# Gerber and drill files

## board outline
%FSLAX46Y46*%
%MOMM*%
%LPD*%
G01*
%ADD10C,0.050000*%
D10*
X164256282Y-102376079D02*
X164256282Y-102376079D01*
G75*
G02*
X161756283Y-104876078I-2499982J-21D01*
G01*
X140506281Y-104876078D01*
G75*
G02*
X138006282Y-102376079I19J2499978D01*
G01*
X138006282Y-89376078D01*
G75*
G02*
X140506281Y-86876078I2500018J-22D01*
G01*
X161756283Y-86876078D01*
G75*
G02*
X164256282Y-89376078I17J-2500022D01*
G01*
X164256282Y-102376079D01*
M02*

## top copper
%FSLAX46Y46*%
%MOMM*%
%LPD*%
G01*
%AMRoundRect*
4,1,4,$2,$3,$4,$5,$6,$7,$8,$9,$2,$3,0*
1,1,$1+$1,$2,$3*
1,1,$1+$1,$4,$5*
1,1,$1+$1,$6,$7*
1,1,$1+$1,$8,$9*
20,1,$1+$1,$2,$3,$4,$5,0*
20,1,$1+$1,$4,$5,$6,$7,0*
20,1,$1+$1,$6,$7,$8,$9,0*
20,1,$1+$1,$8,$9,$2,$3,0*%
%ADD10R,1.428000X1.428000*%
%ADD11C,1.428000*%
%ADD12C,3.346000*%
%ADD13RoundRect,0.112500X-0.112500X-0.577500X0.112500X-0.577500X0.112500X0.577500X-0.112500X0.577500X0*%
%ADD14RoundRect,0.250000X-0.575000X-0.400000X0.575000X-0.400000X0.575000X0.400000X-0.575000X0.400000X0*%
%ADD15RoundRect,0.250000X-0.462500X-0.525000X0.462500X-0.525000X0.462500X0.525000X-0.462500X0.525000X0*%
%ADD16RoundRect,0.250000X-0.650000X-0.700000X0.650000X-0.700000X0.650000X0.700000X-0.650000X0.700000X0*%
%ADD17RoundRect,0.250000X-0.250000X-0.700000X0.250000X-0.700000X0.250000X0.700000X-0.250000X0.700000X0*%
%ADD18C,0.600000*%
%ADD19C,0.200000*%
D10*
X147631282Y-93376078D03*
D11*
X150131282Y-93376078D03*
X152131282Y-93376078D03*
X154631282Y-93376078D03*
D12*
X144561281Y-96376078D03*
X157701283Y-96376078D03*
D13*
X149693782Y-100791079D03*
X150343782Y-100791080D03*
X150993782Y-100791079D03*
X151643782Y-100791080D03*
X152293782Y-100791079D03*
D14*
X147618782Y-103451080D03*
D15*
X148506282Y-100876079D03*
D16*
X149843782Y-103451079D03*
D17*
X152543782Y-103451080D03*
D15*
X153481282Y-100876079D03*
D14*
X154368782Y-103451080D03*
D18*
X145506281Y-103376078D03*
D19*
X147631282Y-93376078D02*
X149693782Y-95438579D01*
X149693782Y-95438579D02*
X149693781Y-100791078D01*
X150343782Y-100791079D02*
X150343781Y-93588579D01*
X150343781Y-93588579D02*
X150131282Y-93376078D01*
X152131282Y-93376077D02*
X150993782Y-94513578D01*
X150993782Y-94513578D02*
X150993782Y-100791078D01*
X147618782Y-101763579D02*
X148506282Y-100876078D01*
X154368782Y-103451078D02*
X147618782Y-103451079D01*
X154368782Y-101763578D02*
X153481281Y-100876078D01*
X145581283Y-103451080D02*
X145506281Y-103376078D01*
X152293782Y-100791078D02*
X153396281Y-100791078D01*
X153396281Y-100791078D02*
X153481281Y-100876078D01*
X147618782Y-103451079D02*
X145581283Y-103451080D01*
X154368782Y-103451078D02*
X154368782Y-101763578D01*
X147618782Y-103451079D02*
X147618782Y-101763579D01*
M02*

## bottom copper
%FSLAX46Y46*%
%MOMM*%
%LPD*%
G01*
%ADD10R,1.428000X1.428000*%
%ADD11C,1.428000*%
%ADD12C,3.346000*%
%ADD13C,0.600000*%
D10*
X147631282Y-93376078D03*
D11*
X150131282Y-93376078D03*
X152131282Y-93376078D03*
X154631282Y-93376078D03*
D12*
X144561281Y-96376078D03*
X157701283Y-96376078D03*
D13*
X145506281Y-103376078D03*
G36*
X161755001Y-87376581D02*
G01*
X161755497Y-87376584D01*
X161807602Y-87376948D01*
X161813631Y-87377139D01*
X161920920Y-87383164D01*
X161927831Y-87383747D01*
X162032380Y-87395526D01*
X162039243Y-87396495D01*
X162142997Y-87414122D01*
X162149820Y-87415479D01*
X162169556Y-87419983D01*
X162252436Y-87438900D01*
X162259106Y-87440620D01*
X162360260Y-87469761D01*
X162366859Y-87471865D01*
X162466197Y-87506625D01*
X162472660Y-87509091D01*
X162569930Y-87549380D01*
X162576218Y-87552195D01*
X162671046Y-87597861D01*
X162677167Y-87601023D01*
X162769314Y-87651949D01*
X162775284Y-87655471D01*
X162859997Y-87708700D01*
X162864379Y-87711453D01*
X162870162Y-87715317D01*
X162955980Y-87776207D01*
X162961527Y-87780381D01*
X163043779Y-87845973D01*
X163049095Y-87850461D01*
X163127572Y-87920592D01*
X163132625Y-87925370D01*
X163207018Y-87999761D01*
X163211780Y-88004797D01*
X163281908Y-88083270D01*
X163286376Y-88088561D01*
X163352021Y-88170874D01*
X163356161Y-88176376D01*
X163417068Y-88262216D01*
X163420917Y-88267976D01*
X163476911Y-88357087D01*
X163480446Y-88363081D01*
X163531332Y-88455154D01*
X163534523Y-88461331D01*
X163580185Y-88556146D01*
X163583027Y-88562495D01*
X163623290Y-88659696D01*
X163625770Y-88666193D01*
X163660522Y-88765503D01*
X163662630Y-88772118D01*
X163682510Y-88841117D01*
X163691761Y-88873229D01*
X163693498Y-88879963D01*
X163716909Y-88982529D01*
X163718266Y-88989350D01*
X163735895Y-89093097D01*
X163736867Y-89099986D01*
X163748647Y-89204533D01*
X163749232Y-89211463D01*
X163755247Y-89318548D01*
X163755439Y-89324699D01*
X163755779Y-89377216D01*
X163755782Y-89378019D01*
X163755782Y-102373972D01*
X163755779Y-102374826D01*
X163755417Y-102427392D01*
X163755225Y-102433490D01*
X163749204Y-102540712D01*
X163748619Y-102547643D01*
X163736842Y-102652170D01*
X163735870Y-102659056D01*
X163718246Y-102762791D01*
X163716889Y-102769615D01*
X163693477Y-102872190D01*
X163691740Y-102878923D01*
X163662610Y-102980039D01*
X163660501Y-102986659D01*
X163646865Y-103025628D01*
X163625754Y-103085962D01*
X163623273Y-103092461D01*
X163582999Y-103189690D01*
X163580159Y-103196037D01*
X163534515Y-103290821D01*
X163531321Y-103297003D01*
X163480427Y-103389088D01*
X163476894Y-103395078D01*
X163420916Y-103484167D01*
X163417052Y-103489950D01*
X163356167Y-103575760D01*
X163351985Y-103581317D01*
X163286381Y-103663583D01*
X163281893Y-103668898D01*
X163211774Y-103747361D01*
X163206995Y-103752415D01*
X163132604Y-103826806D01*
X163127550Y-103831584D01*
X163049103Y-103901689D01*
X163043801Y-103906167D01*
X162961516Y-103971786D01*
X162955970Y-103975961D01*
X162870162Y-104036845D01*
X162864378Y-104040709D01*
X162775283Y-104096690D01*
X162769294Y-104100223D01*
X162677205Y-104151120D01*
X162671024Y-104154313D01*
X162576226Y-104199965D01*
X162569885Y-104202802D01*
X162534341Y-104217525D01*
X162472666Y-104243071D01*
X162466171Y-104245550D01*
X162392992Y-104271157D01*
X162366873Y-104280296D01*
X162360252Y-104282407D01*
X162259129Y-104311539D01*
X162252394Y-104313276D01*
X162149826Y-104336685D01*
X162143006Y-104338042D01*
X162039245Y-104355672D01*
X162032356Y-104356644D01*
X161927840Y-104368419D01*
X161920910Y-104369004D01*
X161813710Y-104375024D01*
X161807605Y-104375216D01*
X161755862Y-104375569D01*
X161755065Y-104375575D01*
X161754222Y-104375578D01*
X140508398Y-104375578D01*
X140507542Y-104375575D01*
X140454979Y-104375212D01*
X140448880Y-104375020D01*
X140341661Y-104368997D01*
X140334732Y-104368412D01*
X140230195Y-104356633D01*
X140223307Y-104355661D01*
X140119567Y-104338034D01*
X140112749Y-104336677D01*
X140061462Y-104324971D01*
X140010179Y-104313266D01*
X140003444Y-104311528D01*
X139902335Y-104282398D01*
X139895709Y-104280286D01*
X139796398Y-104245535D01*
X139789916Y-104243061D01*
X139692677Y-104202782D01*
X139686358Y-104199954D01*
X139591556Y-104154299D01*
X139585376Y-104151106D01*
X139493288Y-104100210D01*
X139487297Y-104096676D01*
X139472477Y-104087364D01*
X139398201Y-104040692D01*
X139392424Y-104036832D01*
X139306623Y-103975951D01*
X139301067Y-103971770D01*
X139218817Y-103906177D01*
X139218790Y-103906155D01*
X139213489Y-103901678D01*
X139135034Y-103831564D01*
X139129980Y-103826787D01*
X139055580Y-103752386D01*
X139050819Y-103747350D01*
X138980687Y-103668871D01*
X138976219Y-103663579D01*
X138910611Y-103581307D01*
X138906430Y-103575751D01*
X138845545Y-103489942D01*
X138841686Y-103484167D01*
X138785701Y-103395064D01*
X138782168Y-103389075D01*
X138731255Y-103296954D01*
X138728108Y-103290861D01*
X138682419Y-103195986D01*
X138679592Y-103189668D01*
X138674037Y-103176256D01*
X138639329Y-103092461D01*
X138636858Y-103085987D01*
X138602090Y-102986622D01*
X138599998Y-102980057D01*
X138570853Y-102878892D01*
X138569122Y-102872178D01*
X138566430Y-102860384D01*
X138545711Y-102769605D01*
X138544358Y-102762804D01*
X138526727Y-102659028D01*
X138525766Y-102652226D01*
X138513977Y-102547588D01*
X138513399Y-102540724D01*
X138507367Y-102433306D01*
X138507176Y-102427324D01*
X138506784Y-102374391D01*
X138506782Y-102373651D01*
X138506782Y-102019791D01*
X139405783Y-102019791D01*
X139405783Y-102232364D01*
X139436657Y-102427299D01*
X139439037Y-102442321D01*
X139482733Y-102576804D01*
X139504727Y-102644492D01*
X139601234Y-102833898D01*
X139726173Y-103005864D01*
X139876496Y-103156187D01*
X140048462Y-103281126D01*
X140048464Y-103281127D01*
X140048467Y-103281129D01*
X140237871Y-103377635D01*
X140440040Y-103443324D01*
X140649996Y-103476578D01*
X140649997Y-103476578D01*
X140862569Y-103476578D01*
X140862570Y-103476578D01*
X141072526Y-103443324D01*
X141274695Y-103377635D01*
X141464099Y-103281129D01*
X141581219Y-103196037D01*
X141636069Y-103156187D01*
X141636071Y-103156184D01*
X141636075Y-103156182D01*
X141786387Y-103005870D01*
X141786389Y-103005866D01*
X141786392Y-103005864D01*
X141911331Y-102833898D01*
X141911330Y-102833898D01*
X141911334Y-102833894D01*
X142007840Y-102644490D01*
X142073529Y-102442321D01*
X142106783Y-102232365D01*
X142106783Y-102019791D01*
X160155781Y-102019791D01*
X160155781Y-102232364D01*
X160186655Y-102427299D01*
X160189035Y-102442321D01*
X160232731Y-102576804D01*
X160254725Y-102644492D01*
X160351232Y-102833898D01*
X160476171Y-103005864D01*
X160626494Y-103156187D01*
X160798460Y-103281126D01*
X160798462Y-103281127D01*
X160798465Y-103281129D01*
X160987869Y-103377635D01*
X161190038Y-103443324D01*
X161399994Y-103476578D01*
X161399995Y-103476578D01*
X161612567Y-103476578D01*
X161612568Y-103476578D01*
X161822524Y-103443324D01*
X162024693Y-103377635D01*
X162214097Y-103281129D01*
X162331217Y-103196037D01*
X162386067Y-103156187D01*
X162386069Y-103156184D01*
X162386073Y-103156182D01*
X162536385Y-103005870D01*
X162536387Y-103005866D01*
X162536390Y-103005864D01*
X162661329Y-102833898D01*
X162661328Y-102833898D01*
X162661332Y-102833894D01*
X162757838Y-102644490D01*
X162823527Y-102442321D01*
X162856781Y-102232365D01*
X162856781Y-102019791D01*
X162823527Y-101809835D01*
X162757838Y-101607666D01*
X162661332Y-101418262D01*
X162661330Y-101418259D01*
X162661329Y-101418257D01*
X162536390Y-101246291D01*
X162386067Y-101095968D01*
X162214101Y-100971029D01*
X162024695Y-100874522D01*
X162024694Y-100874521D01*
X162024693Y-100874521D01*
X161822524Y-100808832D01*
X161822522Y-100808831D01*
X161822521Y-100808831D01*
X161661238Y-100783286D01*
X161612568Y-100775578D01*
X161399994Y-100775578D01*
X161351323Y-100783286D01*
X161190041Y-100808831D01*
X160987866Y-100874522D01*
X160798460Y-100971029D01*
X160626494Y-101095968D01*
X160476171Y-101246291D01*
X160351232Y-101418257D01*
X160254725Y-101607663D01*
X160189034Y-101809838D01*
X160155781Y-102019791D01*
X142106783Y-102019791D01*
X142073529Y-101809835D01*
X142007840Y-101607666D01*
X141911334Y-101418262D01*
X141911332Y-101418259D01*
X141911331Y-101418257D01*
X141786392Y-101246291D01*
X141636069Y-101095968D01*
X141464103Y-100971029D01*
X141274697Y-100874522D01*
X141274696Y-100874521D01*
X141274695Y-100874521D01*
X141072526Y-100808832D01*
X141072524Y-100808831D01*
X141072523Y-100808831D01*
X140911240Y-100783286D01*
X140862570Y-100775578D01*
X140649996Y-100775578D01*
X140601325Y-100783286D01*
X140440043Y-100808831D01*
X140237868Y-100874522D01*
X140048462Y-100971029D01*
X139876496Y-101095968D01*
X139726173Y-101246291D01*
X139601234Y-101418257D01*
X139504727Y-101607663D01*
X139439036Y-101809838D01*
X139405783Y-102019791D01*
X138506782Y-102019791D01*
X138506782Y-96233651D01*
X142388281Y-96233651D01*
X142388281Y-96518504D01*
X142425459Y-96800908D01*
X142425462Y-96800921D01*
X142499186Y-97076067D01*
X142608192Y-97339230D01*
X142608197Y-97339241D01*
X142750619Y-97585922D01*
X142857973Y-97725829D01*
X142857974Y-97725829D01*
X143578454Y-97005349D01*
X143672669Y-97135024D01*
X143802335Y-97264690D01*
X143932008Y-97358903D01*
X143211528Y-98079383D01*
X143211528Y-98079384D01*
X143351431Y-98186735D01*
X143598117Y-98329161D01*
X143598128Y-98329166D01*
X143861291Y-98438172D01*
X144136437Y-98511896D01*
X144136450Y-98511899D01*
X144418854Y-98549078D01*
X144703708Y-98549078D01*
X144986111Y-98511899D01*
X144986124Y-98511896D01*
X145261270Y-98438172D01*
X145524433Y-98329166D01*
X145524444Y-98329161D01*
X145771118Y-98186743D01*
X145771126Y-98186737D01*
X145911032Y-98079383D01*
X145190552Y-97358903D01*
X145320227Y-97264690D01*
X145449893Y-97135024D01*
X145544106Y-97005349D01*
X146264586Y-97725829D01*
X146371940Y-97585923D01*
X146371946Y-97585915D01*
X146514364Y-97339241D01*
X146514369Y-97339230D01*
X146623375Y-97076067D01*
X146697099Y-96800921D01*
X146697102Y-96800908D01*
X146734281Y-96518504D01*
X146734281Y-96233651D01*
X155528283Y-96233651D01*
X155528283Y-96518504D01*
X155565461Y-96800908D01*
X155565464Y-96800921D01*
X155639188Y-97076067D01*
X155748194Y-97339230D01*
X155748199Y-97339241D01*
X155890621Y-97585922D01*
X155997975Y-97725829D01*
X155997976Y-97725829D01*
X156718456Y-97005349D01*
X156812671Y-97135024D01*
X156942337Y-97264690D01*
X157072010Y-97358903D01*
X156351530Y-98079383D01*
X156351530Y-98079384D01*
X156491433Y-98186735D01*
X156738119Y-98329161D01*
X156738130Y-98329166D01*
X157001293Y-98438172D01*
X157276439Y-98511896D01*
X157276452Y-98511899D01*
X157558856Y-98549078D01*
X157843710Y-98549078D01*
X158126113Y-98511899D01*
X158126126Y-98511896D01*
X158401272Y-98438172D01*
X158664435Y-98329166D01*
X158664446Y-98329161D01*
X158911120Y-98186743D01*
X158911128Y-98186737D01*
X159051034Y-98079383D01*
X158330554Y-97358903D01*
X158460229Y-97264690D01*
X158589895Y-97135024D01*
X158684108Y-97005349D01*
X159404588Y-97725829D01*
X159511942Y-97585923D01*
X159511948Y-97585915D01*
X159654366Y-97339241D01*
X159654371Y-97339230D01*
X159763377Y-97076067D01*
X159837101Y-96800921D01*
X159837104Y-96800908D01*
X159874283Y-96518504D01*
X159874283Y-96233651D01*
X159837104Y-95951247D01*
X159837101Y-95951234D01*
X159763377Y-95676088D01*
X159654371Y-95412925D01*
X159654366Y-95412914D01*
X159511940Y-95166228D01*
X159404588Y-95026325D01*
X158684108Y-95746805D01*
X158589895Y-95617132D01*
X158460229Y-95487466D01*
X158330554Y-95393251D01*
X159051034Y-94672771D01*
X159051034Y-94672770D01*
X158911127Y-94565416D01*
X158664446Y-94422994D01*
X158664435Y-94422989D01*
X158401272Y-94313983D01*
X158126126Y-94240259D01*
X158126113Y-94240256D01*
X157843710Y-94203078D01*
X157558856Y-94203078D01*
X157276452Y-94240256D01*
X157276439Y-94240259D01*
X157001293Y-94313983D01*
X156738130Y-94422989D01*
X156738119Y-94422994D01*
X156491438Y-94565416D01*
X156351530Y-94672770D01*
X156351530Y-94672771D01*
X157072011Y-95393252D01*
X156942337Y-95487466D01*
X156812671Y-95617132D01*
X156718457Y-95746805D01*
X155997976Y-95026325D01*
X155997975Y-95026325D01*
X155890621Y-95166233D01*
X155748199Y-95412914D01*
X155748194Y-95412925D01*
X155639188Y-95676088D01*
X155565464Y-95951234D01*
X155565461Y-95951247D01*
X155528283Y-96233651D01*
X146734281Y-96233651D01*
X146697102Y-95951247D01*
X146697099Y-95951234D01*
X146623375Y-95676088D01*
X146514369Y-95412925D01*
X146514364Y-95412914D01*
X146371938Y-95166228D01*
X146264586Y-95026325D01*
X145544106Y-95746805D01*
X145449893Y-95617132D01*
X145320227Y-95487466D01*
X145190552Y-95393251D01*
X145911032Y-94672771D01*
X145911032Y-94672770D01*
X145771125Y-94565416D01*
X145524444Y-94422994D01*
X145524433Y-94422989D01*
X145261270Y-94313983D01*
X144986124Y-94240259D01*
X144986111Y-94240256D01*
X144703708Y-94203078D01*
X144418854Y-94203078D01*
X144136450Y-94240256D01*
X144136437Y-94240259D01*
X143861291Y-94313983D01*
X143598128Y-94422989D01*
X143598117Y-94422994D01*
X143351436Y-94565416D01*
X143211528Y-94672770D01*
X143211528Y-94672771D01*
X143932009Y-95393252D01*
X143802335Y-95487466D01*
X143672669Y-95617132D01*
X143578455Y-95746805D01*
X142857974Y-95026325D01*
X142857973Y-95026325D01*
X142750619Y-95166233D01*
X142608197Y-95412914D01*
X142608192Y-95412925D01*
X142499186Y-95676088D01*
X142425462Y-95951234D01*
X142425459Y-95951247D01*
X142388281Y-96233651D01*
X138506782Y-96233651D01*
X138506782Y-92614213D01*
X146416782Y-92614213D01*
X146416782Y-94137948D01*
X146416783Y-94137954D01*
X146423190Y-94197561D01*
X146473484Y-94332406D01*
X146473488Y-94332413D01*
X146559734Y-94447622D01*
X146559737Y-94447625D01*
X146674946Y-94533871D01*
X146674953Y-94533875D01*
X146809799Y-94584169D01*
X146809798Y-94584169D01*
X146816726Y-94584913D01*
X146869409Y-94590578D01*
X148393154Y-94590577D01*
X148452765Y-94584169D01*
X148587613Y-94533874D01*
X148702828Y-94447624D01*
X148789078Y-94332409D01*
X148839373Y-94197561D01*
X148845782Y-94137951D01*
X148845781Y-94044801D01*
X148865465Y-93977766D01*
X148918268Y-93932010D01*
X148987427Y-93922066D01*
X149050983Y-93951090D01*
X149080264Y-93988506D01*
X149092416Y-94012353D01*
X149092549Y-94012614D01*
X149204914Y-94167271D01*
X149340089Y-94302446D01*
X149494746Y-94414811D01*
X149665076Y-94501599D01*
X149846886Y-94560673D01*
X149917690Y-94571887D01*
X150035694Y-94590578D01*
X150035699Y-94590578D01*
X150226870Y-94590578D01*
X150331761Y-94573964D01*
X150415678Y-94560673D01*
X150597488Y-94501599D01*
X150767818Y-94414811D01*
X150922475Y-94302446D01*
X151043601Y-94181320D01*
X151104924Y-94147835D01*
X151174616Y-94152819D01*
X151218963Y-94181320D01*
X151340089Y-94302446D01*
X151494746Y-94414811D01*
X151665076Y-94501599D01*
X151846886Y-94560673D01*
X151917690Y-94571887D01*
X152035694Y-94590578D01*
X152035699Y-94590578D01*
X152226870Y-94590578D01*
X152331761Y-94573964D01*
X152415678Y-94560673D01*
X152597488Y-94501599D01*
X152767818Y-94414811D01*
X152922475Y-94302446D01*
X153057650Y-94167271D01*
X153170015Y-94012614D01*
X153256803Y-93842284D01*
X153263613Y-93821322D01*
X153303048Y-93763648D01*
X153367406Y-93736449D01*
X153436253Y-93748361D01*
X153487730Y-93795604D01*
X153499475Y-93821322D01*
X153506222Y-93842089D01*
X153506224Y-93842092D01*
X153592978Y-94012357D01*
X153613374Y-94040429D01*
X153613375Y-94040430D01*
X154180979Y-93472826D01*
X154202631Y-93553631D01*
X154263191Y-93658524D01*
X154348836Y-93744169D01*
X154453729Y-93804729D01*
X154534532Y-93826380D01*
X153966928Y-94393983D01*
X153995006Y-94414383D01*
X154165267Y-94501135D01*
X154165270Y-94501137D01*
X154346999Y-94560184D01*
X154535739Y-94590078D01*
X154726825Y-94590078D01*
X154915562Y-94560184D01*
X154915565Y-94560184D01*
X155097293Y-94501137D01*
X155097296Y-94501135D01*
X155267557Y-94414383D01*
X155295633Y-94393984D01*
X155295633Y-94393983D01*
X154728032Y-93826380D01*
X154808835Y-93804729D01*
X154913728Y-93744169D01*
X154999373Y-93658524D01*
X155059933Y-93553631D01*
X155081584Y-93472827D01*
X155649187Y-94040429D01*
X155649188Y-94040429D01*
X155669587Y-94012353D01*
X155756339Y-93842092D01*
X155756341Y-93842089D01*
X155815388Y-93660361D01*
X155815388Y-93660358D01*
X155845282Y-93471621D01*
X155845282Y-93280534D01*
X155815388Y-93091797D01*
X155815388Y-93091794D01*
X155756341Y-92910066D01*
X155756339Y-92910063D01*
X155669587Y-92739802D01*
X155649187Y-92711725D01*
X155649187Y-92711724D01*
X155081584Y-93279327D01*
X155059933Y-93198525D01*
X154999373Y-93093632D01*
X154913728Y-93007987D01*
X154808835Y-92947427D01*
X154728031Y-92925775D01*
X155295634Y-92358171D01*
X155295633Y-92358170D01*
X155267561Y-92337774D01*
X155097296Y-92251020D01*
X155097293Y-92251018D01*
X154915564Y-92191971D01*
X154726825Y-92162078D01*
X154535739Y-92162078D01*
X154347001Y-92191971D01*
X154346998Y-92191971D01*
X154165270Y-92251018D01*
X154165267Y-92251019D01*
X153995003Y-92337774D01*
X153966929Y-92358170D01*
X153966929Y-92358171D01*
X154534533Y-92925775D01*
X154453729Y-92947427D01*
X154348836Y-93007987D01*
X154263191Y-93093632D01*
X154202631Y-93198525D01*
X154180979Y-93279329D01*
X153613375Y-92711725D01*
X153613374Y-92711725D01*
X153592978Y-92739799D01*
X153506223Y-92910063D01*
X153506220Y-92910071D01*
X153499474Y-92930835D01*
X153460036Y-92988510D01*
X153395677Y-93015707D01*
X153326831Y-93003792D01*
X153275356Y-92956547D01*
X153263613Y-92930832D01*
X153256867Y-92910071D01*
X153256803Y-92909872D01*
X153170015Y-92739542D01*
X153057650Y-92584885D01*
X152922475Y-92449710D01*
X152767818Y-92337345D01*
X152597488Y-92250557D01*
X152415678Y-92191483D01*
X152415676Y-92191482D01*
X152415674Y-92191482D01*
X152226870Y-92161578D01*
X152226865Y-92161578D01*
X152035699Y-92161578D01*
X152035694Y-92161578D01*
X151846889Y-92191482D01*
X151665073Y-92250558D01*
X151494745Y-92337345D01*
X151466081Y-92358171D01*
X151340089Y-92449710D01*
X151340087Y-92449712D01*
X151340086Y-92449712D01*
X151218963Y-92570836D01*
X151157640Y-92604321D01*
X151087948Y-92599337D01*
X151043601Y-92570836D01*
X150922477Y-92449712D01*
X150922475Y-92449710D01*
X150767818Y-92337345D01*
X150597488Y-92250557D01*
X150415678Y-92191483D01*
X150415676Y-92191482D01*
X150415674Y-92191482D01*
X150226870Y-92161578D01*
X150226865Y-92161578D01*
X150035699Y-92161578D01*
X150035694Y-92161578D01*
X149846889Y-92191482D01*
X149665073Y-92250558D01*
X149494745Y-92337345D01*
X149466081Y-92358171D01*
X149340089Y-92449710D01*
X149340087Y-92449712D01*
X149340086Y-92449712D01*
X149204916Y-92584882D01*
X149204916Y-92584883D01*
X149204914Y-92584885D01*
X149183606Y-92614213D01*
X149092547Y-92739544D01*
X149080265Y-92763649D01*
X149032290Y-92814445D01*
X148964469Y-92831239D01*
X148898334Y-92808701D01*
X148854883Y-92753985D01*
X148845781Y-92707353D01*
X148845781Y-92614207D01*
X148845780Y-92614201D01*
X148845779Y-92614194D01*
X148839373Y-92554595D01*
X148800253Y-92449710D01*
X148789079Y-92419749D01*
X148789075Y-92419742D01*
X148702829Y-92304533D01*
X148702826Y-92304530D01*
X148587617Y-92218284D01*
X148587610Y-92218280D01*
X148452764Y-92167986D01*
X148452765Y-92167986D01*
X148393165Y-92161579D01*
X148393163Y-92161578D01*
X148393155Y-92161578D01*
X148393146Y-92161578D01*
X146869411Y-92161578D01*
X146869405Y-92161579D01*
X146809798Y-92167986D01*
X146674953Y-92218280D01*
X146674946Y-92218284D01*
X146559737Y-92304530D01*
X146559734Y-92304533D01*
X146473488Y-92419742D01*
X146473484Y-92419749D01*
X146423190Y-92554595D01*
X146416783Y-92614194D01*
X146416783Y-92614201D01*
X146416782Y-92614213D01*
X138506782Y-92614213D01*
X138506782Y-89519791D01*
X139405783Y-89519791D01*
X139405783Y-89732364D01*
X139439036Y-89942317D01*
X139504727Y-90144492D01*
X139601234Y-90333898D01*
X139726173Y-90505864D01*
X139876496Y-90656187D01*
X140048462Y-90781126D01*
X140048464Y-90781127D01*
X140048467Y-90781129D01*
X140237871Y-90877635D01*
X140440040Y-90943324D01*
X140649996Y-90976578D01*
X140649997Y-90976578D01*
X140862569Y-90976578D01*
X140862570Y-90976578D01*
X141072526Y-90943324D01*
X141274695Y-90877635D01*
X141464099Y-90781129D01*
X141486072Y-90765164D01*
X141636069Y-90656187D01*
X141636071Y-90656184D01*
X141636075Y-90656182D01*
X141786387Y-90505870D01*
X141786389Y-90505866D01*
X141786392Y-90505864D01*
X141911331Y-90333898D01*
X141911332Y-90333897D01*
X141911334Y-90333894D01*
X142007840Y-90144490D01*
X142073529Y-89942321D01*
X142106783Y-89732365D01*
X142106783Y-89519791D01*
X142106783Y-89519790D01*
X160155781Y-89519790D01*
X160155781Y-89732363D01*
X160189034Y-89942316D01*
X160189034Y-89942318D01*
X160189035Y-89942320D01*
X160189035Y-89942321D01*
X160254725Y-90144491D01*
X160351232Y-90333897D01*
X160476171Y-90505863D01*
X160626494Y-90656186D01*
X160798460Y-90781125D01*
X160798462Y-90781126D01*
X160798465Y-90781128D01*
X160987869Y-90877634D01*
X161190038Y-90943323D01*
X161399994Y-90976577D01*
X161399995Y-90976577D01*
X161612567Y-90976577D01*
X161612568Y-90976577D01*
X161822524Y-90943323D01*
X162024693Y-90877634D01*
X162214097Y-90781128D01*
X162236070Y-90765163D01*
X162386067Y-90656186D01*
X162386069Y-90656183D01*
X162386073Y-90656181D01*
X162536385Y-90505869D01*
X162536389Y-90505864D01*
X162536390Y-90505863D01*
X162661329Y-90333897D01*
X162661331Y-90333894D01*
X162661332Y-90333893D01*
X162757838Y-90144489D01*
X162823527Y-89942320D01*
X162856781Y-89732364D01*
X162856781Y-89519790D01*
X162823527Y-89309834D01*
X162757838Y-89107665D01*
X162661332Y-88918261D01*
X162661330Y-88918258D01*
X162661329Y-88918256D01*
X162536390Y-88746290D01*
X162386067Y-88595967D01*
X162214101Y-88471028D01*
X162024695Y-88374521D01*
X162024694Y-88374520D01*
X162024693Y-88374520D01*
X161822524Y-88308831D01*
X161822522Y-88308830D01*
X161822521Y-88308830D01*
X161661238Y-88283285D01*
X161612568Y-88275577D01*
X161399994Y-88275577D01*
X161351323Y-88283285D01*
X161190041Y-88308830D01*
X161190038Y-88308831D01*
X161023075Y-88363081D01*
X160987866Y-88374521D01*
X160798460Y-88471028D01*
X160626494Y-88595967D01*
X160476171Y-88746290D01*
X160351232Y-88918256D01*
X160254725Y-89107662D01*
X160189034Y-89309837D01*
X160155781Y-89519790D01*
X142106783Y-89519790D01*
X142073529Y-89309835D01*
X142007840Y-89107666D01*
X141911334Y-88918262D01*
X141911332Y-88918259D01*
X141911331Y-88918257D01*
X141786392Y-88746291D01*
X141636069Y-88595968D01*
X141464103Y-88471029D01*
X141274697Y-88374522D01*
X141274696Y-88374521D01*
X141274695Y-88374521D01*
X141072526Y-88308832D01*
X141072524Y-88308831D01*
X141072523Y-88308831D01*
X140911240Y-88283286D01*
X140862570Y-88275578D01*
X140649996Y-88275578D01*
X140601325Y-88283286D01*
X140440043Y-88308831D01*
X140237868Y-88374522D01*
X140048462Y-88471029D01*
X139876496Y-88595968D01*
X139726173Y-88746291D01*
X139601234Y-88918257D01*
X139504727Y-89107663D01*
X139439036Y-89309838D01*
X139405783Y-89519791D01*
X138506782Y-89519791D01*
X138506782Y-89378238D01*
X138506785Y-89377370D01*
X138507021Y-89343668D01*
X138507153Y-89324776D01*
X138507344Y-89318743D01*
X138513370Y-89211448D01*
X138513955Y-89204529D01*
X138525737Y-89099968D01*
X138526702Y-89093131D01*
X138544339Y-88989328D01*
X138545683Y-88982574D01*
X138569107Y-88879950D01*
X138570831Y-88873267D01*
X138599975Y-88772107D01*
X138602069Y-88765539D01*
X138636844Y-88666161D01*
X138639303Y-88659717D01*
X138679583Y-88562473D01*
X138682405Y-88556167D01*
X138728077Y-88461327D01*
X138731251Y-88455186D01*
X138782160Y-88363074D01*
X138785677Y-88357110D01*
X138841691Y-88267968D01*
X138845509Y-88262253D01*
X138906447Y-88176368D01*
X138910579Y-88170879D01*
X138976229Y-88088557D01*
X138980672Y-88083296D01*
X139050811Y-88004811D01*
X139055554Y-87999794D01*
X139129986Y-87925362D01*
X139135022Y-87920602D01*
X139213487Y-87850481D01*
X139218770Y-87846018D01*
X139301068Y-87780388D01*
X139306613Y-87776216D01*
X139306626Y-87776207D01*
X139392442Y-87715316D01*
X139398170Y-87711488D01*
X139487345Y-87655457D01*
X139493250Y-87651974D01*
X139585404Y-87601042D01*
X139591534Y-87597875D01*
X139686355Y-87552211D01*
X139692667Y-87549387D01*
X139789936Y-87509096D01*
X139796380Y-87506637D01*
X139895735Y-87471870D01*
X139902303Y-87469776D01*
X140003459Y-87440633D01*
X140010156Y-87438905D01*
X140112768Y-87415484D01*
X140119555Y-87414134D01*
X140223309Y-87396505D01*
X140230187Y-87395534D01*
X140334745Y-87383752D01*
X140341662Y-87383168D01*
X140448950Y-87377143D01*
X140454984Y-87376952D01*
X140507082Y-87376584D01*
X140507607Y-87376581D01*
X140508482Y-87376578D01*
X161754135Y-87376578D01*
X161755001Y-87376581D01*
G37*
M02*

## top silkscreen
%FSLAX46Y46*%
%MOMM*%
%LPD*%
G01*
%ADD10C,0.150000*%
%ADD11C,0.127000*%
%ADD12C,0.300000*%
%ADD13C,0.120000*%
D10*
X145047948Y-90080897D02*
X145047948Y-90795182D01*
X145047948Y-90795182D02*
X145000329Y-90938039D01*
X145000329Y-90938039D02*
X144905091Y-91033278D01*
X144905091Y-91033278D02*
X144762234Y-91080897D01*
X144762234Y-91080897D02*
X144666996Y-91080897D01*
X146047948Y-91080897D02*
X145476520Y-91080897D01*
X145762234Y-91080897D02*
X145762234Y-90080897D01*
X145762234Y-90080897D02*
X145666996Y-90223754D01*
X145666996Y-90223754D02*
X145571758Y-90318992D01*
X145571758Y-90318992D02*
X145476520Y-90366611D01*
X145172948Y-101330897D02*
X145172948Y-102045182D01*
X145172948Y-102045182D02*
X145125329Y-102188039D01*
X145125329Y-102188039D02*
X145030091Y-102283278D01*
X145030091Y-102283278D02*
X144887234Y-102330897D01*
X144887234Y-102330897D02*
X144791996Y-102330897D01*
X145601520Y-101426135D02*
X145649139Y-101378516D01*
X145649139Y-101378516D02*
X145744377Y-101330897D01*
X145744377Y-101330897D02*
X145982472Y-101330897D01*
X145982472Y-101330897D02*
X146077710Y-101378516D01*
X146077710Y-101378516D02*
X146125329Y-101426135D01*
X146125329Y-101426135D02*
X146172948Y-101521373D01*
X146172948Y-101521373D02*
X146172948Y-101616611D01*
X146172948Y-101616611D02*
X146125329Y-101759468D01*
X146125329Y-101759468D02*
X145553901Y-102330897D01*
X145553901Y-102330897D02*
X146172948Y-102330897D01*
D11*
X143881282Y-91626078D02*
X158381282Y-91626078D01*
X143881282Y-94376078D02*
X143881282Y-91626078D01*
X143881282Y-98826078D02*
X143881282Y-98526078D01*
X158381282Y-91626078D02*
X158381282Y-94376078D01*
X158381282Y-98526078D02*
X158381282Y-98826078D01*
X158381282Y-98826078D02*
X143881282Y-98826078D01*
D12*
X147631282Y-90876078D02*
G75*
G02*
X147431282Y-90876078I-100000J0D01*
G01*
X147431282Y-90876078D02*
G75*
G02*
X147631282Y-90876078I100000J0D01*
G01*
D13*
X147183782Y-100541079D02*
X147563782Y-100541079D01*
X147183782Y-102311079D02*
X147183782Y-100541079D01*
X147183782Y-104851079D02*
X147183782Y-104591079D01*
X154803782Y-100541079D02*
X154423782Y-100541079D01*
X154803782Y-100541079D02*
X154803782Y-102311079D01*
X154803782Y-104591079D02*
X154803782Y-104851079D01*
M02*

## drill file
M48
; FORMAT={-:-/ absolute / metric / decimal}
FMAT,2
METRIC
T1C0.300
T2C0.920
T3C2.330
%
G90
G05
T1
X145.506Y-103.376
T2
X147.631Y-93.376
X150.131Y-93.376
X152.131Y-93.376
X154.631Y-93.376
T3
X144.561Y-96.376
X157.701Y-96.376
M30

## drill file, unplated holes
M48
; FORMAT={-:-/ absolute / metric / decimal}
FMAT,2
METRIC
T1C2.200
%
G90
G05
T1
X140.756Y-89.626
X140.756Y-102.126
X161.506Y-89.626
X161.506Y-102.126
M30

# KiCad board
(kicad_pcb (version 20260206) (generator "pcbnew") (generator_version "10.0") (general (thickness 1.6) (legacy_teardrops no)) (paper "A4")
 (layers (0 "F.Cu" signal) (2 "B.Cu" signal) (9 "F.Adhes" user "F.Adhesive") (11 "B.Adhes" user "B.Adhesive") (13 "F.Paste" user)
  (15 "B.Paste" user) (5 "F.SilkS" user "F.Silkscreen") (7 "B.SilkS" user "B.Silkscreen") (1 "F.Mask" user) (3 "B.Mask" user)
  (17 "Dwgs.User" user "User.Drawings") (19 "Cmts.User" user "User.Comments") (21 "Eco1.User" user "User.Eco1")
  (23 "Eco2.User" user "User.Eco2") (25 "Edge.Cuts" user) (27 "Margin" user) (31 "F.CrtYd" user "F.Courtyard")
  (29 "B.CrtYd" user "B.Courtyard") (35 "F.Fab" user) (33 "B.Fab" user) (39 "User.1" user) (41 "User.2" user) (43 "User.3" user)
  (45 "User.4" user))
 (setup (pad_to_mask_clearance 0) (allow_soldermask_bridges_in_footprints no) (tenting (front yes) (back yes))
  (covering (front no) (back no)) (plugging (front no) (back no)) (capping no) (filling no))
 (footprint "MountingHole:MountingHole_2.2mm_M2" (layer "F.Cu") (at 140.756283 89.626078 180)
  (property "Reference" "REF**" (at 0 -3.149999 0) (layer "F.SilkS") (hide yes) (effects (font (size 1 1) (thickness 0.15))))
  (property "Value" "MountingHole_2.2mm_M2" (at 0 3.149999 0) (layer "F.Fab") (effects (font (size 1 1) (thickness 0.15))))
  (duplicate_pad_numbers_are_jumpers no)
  (pad "" np_thru_hole circle (at 0 0 180) (size 2.2 2.2) (drill 2.2) (layers "*.Cu" "*.Mask")))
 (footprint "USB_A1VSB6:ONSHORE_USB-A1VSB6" (layer "F.Cu") (at 151.131282 96.376078)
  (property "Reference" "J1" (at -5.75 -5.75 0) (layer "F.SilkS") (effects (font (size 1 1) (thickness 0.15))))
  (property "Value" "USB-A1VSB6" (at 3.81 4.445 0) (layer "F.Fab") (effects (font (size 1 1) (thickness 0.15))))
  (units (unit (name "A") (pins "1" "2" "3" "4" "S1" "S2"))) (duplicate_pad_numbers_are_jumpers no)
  (fp_line (start -7.25 -4.75) (end 7.25 -4.75) (stroke (width 0.127) (type solid)) (layer "F.SilkS"))
  (fp_line (start -7.25 -2) (end -7.25 -4.75) (stroke (width 0.127) (type solid)) (layer "F.SilkS"))
  (fp_line (start -7.25 2.45) (end -7.25 2.15) (stroke (width 0.127) (type solid)) (layer "F.SilkS"))
  (fp_line (start 7.25 -4.75) (end 7.25 -2) (stroke (width 0.127) (type solid)) (layer "F.SilkS"))
  (fp_line (start 7.25 2.15) (end 7.25 2.45) (stroke (width 0.127) (type solid)) (layer "F.SilkS"))
  (fp_line (start 7.25 2.45) (end -7.25 2.45) (stroke (width 0.127) (type solid)) (layer "F.SilkS"))
  (fp_circle (center -3.6 -5.5) (end -3.5 -5.5) (stroke (width 0.3) (type solid)) (fill no) (layer "F.SilkS"))
  (pad "1" thru_hole rect (at -3.5 -3) (size 1.428 1.428) (drill 0.92) (layers "*.Cu" "*.Mask") (remove_unused_layers no)
   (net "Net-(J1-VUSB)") (solder_mask_margin 0.102))
  (pad "2" thru_hole circle (at -1 -3) (size 1.428 1.428) (drill 0.92) (layers "*.Cu" "*.Mask") (remove_unused_layers no)
   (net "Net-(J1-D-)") (solder_mask_margin 0.102))
  (pad "3" thru_hole circle (at 1 -3) (size 1.428 1.428) (drill 0.92) (layers "*.Cu" "*.Mask") (remove_unused_layers no) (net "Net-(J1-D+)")
   (solder_mask_margin 0.102))
  (pad "4" thru_hole circle (at 3.5 -3) (size 1.428 1.428) (drill 0.92) (layers "*.Cu" "*.Mask") (remove_unused_layers no)
   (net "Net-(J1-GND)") (solder_mask_margin 0.102))
  (pad "S1" thru_hole circle (at -6.570001 0) (size 3.346 3.346) (drill 2.33) (layers "*.Cu" "*.Mask") (remove_unused_layers no)
   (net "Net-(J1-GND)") (solder_mask_margin 0.102))
  (pad "S2" thru_hole circle (at 6.570001 0) (size 3.346 3.346) (drill 2.33) (layers "*.Cu" "*.Mask") (remove_unused_layers no)
   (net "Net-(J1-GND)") (solder_mask_margin 0.102)))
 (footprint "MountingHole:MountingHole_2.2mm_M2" (layer "F.Cu") (at 140.756283 102.126078 180)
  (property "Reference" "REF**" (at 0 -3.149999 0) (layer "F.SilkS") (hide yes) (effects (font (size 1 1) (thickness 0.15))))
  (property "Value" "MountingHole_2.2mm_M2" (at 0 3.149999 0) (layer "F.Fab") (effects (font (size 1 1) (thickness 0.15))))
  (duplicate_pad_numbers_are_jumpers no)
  (pad "" np_thru_hole circle (at 0 0 180) (size 2.2 2.2) (drill 2.2) (layers "*.Cu" "*.Mask")))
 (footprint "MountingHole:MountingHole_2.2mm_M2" (layer "F.Cu") (at 161.506281 89.626077 180)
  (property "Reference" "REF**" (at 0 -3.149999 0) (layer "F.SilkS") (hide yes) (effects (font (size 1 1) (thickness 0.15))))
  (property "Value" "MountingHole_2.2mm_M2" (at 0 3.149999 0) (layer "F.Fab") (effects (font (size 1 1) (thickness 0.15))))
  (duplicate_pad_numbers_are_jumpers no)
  (pad "" np_thru_hole circle (at 0 0 180) (size 2.2 2.2) (drill 2.2) (layers "*.Cu" "*.Mask")))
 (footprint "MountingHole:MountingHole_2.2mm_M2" (layer "F.Cu") (at 161.506281 102.126078 180)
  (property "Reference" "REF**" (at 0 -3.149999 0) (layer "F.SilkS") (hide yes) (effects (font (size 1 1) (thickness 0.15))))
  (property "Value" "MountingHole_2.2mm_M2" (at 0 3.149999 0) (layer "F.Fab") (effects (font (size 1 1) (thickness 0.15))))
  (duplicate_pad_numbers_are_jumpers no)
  (pad "" np_thru_hole circle (at 0 0 180) (size 2.2 2.2) (drill 2.2) (layers "*.Cu" "*.Mask")))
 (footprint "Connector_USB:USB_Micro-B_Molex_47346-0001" (layer "F.Cu") (at 150.993782 102.251079)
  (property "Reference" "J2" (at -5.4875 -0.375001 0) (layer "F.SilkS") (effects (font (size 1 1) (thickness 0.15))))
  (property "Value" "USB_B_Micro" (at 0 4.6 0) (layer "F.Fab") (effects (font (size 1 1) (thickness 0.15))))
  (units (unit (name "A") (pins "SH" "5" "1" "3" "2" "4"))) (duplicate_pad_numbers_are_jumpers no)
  (fp_line (start -3.81 -1.71) (end -3.43 -1.71) (stroke (width 0.12) (type solid)) (layer "F.SilkS"))
  (fp_line (start -3.81 0.06) (end -3.81 -1.71) (stroke (width 0.12) (type solid)) (layer "F.SilkS"))
  (fp_line (start -3.81 2.6) (end -3.81 2.34) (stroke (width 0.12) (type solid)) (layer "F.SilkS"))
  (fp_line (start 3.81 -1.71) (end 3.43 -1.71) (stroke (width 0.12) (type solid)) (layer "F.SilkS"))
  (fp_line (start 3.81 -1.71) (end 3.81 0.06) (stroke (width 0.12) (type solid)) (layer "F.SilkS"))
  (fp_line (start 3.81 2.34) (end 3.81 2.6) (stroke (width 0.12) (type solid)) (layer "F.SilkS"))
  (pad "1" smd roundrect (at -1.3 -1.46) (size 0.45 1.38) (layers "F.Cu" "F.Mask" "F.Paste") (roundrect_rratio 0.25) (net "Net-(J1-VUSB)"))
  (pad "2" smd roundrect (at -0.65 -1.459999) (size 0.45 1.38) (layers "F.Cu" "F.Mask" "F.Paste") (roundrect_rratio 0.25)
   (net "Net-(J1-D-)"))
  (pad "3" smd roundrect (at 0 -1.46) (size 0.45 1.38) (layers "F.Cu" "F.Mask" "F.Paste") (roundrect_rratio 0.25) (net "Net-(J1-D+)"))
  (pad "4" smd roundrect (at 0.65 -1.459999) (size 0.45 1.38) (layers "F.Cu" "F.Mask" "F.Paste") (roundrect_rratio 0.25)
   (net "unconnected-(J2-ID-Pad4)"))
  (pad "5" smd roundrect (at 1.3 -1.46) (size 0.45 1.38) (layers "F.Cu" "F.Mask" "F.Paste") (roundrect_rratio 0.25) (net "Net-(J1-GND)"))
  (pad "SH" smd roundrect (at -3.375 1.200001) (size 1.65 1.3) (layers "F.Cu" "F.Mask" "F.Paste") (roundrect_rratio 0.1923076923)
   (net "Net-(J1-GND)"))
  (pad "SH" smd roundrect (at -2.4875 -1.375) (size 1.425 1.55) (layers "F.Cu" "F.Mask" "F.Paste") (roundrect_rratio 0.1754385965)
   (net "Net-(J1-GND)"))
  (pad "SH" smd roundrect (at -1.15 1.2) (size 1.8 1.9) (layers "F.Cu" "F.Mask" "F.Paste") (roundrect_rratio 0.1388888889)
   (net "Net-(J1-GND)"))
  (pad "SH" smd roundrect (at 1.55 1.200001) (size 1 1.9) (layers "F.Cu" "F.Mask" "F.Paste") (roundrect_rratio 0.25) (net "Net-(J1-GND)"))
  (pad "SH" smd roundrect (at 2.4875 -1.375) (size 1.425 1.55) (layers "F.Cu" "F.Mask" "F.Paste") (roundrect_rratio 0.1754385965)
   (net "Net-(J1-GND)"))
  (pad "SH" smd roundrect (at 3.375 1.200001) (size 1.65 1.3) (layers "F.Cu" "F.Mask" "F.Paste") (roundrect_rratio 0.1923076923)
   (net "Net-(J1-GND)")))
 (gr_poly
  (pts
   (arc (start 164.256282 102.376079) (mid 163.524049 104.143846) (end 161.756283 104.876078))
   (arc (start 140.506281 104.876078) (mid 138.738515 104.143846) (end 138.006282 102.376079))
   (arc (start 138.006282 89.376078) (mid 138.738515 87.608311) (end 140.506281 86.876078))
   (arc (start 161.756283 86.876078) (mid 163.524049 87.608311) (end 164.256282 89.376078)))
  (stroke (width 0.05) (type solid)) (fill no) (layer "Edge.Cuts"))
 (segment (start 147.631282 93.376078) (end 149.693782 95.438579) (width 0.2) (layer "F.Cu") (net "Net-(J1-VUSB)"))
 (segment (start 149.693782 95.438579) (end 149.693781 100.791078) (width 0.2) (layer "F.Cu") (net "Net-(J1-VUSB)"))
 (segment (start 150.343782 100.791079) (end 150.343781 93.588579) (width 0.2) (layer "F.Cu") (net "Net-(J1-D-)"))
 (segment (start 150.343781 93.588579) (end 150.131282 93.376078) (width 0.2) (layer "F.Cu") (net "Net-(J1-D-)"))
 (segment (start 152.131282 93.376077) (end 150.993782 94.513578) (width 0.2) (layer "F.Cu") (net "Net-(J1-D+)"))
 (segment (start 150.993782 94.513578) (end 150.993782 100.791078) (width 0.2) (layer "F.Cu") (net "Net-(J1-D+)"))
 (segment (start 147.618782 101.763579) (end 148.506282 100.876078) (width 0.2) (layer "F.Cu") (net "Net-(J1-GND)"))
 (segment (start 154.368782 103.451078) (end 147.618782 103.451079) (width 0.2) (layer "F.Cu") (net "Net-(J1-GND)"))
 (segment (start 154.368782 101.763578) (end 153.481281 100.876078) (width 0.2) (layer "F.Cu") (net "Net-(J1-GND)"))
 (segment (start 145.581283 103.45108) (end 145.506281 103.376078) (width 0.2) (layer "F.Cu") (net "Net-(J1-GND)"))
 (segment (start 152.293782 100.791078) (end 153.396281 100.791078) (width 0.2) (layer "F.Cu") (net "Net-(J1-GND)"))
 (segment (start 153.396281 100.791078) (end 153.481281 100.876078) (width 0.2) (layer "F.Cu") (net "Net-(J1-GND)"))
 (segment (start 147.618782 103.451079) (end 145.581283 103.45108) (width 0.2) (layer "F.Cu") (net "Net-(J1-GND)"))
 (segment (start 154.368782 103.451078) (end 154.368782 101.763578) (width 0.2) (layer "F.Cu") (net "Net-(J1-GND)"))
 (segment (start 147.618782 103.451079) (end 147.618782 101.763579) (width 0.2) (layer "F.Cu") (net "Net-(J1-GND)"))
 (via (at 145.506281 103.376078) (size 0.6) (drill 0.3) (layers "F.Cu" "B.Cu") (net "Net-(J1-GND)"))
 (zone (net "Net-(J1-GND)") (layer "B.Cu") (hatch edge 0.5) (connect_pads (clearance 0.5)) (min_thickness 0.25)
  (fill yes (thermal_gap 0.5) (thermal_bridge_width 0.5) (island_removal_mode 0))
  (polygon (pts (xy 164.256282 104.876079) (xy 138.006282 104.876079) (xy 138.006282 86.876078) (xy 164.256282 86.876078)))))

